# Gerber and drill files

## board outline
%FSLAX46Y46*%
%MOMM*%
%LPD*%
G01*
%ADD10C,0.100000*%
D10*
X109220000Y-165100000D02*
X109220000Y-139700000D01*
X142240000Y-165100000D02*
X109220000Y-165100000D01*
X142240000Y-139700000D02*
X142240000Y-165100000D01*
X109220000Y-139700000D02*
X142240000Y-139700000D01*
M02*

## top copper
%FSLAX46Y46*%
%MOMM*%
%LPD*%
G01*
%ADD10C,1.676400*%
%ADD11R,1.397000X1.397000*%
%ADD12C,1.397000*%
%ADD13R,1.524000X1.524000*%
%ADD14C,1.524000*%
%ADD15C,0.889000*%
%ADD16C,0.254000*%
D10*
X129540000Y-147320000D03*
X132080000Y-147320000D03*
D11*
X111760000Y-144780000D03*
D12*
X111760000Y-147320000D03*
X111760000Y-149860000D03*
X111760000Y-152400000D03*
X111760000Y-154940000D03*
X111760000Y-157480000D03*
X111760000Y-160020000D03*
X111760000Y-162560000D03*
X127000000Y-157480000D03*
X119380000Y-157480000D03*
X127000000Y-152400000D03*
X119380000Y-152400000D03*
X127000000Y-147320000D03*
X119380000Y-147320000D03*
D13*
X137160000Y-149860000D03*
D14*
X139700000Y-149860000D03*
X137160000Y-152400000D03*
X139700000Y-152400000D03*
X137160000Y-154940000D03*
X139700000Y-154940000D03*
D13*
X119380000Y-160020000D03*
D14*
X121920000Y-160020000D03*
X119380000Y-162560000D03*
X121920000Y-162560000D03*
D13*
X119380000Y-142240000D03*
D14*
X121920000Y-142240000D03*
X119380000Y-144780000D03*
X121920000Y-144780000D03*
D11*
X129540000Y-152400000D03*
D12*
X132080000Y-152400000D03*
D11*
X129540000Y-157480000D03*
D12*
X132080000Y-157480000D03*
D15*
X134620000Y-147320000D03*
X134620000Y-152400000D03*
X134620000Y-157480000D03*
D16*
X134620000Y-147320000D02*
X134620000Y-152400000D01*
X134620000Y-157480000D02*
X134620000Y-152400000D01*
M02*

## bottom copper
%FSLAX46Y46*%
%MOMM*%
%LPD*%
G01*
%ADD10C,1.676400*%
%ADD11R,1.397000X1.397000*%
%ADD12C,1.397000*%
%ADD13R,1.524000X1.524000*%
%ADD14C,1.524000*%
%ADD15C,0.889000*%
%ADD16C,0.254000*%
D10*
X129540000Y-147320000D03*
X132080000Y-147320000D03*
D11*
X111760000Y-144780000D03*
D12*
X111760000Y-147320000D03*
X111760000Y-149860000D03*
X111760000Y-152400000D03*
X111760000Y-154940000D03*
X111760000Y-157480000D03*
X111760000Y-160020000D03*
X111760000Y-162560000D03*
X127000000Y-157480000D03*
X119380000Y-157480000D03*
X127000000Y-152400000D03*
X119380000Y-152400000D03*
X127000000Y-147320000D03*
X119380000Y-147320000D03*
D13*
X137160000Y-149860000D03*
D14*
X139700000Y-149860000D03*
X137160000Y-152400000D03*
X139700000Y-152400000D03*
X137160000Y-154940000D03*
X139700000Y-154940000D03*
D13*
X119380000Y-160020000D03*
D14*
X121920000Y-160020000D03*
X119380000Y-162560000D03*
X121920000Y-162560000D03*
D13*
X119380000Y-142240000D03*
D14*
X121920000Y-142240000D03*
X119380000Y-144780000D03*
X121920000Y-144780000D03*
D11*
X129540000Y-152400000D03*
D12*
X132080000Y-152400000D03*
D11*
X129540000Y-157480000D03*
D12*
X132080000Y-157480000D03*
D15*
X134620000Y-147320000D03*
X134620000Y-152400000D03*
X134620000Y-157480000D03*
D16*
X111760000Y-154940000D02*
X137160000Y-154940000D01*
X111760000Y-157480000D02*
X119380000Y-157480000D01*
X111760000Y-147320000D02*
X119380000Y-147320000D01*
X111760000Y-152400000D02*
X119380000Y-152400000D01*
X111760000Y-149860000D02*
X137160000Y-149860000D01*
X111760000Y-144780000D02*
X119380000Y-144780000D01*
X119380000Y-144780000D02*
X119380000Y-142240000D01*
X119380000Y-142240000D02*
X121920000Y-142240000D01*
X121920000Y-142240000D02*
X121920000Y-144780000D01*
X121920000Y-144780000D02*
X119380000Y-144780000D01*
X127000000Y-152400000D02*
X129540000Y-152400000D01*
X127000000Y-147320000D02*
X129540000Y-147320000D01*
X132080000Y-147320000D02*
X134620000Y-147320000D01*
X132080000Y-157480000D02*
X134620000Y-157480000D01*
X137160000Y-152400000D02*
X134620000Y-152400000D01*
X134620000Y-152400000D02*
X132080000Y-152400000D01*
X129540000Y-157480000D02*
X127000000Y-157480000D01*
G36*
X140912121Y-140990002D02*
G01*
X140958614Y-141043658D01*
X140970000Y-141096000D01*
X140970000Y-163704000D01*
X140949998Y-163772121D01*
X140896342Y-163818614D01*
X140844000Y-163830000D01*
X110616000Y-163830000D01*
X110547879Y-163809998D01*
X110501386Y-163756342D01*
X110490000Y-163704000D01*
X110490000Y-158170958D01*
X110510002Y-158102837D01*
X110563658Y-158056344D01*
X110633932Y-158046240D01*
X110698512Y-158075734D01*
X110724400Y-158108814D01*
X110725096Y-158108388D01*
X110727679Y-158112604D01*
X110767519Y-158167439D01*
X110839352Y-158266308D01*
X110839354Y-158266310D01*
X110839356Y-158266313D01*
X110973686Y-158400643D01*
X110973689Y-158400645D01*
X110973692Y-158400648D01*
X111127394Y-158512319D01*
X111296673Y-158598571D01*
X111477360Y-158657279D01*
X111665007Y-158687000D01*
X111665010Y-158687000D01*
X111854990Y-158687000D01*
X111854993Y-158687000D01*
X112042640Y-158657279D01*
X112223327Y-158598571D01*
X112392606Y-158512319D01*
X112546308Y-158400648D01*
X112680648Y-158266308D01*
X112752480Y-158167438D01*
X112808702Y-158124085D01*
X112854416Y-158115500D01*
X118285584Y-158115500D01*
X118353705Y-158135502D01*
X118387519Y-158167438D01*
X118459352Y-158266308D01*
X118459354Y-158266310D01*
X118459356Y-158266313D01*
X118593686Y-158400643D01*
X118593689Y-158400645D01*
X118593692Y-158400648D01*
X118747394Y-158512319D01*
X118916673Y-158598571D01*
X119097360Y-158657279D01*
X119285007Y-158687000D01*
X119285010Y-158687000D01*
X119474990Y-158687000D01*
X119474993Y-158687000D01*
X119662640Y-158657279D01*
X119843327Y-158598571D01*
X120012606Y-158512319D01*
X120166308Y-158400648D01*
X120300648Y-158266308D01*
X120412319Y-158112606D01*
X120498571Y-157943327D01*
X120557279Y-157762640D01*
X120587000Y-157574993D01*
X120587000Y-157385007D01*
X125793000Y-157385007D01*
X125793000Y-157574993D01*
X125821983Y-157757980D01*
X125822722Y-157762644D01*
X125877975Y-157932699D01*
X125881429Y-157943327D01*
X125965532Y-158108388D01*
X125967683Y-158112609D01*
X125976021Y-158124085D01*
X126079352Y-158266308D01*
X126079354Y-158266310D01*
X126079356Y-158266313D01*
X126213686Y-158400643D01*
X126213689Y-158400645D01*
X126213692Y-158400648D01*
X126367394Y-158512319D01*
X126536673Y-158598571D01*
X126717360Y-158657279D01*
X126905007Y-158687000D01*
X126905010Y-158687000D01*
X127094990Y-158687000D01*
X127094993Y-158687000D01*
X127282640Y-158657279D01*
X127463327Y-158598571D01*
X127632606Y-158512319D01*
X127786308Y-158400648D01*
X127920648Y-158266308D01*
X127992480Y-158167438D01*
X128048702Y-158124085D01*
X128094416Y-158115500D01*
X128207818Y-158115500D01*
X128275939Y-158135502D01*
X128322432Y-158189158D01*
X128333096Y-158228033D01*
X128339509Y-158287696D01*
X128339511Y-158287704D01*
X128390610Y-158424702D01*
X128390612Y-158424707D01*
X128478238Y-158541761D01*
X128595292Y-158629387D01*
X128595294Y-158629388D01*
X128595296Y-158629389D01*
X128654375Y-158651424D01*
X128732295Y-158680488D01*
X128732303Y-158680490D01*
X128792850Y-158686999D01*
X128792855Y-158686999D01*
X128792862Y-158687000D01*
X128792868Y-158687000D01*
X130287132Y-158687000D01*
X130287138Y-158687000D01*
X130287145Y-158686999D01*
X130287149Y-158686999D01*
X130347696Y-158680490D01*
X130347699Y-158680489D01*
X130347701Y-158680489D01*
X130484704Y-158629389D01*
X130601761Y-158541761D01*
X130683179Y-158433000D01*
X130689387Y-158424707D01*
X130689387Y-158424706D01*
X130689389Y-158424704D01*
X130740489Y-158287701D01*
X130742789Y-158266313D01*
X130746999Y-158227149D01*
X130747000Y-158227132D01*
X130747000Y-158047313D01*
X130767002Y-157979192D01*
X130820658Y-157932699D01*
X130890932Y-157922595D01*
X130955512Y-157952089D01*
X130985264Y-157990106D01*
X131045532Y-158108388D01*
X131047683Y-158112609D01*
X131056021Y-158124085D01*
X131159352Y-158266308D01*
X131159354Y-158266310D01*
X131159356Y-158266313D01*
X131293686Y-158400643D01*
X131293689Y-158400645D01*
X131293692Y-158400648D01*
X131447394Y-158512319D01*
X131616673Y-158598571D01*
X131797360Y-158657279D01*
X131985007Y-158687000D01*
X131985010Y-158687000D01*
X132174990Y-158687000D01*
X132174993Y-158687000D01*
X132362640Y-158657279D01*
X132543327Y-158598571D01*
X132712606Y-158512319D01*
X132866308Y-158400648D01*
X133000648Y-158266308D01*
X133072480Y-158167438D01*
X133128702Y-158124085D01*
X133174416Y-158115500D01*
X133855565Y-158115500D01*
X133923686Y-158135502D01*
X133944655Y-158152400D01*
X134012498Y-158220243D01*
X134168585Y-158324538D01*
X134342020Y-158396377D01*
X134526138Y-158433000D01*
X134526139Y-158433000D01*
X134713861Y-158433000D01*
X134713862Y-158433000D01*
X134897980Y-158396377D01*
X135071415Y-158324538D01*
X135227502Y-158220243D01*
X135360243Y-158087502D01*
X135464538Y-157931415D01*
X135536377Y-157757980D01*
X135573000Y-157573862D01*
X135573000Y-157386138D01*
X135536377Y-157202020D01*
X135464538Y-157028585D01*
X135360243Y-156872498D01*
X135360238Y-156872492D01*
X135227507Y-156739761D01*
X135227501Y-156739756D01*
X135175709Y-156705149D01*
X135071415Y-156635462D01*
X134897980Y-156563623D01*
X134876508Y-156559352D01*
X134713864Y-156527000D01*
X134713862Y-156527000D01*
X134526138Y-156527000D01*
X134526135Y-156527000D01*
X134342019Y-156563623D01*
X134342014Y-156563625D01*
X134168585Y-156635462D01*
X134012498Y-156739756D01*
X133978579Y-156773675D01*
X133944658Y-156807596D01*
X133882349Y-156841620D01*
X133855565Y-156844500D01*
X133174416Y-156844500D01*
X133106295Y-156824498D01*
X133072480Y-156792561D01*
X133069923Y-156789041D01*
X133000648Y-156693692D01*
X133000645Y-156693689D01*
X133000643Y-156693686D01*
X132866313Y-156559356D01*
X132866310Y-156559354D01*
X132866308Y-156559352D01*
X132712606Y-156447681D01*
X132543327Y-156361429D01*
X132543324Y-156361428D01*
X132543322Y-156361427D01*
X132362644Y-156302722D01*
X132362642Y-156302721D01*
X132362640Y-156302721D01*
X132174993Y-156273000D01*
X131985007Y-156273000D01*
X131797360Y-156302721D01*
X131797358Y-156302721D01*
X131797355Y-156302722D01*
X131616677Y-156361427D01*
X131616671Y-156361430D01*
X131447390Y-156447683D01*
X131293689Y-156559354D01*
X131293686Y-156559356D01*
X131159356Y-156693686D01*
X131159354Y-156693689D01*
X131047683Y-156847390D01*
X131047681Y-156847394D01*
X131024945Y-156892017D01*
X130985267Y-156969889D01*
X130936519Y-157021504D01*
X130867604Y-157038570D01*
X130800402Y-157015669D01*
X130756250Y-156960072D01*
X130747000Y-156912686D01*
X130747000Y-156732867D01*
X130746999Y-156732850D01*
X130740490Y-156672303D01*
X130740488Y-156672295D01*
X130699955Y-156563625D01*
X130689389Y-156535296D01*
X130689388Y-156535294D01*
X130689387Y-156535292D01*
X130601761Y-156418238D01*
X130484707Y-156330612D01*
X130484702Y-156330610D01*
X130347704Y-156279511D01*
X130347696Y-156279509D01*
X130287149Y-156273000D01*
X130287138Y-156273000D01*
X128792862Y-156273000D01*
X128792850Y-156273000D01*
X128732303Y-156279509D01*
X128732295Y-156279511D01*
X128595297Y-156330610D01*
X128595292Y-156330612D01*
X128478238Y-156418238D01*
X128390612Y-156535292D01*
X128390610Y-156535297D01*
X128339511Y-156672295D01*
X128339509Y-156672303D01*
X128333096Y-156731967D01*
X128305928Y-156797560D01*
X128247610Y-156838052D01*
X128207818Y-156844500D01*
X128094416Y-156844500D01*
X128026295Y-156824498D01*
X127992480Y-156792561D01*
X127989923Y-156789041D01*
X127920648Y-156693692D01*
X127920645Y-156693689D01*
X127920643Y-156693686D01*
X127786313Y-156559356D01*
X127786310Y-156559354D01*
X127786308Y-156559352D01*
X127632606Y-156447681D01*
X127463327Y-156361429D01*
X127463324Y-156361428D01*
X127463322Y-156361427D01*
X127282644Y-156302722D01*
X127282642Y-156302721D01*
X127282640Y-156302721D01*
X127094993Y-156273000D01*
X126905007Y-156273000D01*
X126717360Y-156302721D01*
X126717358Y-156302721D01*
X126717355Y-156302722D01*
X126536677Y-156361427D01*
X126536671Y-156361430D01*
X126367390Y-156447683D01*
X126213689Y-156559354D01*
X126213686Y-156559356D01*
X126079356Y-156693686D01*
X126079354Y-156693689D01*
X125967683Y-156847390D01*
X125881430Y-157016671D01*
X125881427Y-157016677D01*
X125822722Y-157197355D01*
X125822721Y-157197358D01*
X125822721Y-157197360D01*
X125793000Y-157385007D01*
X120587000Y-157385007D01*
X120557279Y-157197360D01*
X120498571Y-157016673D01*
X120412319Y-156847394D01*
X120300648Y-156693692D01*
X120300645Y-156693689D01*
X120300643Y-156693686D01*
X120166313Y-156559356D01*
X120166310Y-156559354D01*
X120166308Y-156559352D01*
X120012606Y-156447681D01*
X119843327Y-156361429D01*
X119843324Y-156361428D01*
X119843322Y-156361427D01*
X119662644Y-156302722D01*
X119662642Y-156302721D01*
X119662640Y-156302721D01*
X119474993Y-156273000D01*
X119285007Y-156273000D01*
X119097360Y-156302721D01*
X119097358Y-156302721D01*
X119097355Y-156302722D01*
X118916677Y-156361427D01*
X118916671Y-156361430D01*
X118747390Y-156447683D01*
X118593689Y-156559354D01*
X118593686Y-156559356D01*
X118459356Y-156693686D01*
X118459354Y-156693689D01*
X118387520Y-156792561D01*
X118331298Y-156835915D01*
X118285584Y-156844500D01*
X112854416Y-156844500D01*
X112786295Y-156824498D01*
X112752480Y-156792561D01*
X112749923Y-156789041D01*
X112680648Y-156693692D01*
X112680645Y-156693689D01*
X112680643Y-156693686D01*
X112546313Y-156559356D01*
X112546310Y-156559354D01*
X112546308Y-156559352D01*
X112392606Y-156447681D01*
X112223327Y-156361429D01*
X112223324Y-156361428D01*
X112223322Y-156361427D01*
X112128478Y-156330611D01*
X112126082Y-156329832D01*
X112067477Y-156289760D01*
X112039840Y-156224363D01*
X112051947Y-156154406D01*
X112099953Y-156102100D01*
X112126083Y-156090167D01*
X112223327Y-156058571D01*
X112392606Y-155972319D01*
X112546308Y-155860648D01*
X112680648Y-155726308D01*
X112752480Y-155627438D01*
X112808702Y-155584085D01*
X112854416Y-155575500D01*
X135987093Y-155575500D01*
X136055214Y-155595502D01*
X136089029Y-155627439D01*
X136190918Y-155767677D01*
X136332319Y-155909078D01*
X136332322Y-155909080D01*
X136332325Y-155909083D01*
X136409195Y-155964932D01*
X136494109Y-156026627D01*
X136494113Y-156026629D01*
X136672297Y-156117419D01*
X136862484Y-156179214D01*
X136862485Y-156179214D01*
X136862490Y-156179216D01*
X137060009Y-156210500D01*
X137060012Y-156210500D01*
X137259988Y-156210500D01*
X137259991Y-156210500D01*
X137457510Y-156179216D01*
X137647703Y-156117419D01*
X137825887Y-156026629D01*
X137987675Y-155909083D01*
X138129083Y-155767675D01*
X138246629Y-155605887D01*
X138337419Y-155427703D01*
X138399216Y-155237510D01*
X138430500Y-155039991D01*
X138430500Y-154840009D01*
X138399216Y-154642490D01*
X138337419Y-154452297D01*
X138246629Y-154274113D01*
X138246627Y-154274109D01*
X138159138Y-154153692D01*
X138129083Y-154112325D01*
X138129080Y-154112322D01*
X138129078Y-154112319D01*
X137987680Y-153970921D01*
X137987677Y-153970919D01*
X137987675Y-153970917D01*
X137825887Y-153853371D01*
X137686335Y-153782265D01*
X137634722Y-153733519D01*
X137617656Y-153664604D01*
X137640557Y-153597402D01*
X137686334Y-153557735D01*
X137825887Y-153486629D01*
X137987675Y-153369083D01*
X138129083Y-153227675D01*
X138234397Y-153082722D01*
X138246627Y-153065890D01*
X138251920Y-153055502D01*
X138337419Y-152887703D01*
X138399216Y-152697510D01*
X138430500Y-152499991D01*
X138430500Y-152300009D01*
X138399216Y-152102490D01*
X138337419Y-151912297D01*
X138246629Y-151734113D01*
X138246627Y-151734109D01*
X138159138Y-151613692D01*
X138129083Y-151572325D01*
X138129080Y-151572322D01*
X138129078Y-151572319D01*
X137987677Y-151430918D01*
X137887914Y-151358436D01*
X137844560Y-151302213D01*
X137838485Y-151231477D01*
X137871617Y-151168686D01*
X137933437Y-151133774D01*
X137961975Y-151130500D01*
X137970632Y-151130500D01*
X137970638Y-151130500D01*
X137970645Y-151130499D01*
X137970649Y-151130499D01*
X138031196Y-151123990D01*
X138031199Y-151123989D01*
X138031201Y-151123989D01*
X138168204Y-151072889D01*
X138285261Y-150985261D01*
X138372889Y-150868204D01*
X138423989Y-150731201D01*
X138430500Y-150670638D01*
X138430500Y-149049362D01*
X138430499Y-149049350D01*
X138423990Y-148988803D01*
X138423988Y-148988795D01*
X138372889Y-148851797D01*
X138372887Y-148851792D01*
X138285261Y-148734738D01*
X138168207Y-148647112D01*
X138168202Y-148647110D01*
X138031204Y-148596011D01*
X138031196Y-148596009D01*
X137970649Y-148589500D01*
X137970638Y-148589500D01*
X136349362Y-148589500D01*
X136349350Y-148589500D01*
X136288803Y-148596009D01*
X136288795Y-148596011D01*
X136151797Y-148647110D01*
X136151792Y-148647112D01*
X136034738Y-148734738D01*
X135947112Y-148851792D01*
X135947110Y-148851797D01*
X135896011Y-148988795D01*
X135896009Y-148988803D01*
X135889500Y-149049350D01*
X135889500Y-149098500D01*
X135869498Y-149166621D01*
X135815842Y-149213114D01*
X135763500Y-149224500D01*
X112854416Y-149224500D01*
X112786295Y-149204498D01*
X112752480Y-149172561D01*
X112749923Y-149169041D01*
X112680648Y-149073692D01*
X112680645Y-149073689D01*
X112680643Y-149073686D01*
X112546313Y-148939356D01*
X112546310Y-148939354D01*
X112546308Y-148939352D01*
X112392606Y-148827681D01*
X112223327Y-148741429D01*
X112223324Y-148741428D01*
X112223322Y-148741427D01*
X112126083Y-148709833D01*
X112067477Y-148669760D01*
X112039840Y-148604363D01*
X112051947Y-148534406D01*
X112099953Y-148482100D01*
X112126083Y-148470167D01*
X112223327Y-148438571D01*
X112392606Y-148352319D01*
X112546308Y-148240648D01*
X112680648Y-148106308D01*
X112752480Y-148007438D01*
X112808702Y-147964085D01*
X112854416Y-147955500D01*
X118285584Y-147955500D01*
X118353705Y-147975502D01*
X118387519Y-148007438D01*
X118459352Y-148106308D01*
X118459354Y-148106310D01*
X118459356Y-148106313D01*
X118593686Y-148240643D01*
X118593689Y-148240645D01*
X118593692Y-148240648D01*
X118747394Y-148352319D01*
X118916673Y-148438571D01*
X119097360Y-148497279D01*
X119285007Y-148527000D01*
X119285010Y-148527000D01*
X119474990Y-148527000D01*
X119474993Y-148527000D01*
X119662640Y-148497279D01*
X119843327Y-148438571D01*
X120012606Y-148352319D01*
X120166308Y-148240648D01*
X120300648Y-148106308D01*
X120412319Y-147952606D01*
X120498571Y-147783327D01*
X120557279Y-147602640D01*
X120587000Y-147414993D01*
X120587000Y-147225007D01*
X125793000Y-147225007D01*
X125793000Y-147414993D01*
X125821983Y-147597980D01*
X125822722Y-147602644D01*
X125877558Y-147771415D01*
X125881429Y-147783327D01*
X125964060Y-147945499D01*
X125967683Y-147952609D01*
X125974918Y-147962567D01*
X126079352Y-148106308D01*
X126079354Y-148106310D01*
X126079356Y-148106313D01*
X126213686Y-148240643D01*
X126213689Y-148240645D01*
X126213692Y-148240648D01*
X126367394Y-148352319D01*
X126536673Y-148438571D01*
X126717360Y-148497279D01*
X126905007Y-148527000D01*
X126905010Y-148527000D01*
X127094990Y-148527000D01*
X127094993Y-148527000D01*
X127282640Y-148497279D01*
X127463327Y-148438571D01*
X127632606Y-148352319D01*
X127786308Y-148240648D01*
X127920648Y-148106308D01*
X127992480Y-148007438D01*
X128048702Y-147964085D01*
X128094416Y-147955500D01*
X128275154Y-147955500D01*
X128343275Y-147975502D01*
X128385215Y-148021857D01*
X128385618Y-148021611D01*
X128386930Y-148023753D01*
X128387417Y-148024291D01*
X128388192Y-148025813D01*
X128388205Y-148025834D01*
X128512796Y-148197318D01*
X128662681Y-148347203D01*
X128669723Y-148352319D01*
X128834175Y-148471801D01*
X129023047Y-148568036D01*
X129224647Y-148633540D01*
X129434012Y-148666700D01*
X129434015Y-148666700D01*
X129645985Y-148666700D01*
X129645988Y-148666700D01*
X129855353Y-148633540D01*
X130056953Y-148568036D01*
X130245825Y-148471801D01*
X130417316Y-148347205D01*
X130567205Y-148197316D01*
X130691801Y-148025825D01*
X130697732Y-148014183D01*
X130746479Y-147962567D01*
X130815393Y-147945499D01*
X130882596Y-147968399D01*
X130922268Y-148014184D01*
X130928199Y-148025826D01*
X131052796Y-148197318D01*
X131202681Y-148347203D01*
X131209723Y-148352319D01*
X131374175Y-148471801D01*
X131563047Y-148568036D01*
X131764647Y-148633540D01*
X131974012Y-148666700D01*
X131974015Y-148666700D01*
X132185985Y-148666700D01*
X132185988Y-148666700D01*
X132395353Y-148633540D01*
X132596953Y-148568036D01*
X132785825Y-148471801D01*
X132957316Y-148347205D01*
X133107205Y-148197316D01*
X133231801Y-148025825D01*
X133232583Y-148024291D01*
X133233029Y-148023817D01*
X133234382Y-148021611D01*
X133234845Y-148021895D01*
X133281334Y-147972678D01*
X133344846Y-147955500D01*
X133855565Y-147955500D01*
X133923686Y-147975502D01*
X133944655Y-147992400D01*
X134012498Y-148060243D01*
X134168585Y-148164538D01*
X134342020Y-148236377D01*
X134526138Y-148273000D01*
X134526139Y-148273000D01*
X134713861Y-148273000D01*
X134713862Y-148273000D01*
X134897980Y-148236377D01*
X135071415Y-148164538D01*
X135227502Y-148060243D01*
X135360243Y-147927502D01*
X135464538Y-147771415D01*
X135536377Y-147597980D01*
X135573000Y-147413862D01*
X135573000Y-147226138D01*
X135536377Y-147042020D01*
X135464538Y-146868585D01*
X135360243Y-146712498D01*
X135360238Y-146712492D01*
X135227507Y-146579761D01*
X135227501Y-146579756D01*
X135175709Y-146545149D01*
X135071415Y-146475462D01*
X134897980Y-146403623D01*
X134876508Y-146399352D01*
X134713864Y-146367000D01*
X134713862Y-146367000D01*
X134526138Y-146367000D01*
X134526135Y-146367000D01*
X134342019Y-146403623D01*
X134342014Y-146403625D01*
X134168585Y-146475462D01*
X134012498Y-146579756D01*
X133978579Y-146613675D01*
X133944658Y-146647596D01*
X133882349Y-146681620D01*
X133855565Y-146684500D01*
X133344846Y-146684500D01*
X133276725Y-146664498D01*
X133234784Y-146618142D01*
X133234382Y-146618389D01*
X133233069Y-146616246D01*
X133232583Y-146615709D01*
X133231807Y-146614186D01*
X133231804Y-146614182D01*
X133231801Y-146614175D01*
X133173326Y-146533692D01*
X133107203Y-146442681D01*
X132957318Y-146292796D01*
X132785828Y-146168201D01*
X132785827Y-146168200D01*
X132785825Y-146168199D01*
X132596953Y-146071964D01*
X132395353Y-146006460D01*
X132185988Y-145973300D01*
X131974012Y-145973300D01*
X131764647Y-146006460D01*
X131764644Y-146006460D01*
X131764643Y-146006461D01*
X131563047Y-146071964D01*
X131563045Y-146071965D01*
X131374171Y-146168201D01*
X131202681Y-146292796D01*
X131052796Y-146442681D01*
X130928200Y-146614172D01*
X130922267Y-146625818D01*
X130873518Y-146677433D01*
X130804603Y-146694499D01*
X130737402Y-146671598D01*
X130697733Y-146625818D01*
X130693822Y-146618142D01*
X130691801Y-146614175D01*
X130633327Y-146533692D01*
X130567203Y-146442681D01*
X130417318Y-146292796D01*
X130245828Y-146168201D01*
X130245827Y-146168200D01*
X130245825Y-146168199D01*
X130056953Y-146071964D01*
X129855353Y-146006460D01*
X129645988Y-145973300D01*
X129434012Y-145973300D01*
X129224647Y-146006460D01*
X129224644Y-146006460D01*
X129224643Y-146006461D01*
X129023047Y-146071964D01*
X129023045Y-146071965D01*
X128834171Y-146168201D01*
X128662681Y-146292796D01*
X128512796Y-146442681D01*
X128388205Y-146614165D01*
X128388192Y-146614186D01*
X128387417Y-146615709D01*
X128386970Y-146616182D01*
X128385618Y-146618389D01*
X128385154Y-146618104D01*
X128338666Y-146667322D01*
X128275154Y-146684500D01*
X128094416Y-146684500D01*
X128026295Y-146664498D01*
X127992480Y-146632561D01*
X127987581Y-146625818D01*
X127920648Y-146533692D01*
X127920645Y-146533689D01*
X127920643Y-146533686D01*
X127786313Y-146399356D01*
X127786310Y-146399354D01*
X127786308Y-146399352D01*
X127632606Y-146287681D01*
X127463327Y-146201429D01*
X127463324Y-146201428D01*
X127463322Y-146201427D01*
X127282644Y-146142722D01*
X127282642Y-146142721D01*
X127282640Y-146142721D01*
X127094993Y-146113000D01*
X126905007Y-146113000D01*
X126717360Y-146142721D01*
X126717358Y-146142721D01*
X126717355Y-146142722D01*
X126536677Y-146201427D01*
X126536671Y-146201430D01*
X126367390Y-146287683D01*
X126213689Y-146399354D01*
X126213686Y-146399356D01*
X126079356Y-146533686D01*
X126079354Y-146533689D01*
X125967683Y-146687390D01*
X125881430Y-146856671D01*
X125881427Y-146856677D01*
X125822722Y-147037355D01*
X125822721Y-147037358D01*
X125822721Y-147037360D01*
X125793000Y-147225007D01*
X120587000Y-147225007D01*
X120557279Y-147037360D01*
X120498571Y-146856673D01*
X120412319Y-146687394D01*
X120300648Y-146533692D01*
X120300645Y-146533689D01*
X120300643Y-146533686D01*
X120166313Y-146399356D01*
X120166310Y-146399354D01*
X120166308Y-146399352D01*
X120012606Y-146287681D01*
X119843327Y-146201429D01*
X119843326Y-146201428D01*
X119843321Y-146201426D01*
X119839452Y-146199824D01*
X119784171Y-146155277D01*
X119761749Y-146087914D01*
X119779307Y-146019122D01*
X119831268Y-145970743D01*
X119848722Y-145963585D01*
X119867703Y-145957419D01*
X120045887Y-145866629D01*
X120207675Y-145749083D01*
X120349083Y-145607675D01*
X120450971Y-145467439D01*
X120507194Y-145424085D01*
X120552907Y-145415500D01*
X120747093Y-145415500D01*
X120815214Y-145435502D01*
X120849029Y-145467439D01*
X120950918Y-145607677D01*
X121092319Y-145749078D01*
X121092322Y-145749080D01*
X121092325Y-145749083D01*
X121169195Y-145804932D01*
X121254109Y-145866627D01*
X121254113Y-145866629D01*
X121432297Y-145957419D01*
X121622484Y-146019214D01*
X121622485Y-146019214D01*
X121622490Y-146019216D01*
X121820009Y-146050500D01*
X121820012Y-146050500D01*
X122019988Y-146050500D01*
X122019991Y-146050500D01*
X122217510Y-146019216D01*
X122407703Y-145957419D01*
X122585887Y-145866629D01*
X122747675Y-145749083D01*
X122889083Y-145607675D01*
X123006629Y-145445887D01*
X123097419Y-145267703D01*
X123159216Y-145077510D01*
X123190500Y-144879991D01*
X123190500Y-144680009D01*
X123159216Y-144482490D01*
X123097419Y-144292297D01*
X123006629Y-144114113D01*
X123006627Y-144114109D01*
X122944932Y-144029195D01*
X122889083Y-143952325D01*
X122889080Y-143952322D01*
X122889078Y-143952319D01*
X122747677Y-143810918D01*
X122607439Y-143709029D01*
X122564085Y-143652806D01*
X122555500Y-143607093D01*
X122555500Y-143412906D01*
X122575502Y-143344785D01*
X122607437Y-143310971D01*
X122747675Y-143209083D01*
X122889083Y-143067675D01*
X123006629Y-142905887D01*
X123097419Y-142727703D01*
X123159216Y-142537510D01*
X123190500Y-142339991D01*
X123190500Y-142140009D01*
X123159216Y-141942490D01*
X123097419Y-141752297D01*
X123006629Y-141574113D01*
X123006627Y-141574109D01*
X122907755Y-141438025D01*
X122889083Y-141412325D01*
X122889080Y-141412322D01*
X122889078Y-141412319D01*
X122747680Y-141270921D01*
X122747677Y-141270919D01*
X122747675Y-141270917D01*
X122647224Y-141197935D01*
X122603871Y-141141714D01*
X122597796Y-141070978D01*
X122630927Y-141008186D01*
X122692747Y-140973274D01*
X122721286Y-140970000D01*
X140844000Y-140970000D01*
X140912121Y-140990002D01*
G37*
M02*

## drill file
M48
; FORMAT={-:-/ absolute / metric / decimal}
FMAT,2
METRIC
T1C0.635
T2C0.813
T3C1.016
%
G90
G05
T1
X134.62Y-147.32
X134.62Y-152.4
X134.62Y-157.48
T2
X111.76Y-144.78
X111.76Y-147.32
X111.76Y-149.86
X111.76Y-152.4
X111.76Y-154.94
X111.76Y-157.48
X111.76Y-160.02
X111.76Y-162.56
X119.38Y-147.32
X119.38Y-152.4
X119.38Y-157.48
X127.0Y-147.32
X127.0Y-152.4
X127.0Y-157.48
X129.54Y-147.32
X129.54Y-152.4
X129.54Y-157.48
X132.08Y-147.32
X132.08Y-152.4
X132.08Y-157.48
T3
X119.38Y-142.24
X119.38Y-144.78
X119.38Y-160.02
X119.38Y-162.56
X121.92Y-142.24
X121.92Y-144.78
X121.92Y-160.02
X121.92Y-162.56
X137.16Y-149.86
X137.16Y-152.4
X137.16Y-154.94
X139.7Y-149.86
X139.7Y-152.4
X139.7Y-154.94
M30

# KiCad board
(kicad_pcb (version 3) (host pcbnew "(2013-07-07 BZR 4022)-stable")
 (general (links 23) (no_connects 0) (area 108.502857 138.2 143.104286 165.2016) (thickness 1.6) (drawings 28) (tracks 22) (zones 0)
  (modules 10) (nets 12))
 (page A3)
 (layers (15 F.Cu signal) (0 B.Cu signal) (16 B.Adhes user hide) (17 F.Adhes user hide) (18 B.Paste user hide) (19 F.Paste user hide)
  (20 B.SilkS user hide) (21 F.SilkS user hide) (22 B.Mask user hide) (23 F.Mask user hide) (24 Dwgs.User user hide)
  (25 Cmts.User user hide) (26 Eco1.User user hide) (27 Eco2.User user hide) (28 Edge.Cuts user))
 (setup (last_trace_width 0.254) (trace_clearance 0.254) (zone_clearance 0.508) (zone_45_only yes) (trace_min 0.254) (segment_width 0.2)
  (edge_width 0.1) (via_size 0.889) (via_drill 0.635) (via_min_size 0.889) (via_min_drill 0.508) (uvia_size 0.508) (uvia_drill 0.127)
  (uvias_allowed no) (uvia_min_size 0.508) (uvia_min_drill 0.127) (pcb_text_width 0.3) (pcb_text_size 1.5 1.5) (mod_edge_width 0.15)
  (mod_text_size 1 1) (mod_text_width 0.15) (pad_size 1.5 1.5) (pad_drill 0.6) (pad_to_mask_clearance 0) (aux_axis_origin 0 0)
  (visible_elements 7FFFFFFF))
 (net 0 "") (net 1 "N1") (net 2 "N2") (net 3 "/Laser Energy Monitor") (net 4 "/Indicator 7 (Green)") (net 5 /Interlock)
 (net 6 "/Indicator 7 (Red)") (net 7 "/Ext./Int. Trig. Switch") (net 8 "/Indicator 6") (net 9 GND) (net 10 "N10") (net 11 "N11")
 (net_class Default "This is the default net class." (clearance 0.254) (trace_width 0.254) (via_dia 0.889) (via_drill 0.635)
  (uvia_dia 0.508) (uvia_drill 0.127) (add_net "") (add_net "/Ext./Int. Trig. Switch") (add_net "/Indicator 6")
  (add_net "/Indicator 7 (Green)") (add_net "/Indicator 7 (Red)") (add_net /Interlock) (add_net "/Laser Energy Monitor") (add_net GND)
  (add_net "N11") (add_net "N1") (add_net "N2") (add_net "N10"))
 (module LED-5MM (layer F.Cu) (at 130.81 147.32)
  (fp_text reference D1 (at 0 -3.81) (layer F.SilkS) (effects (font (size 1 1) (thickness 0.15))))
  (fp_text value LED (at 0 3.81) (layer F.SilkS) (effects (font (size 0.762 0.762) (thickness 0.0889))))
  (pad 1 thru_hole circle (at -1.27 0) (size 1.6764 1.6764) (drill 0.8128) (layers *.Cu *.Mask F.SilkS) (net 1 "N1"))
  (pad 2 thru_hole circle (at 1.27 0) (size 1.6764 1.6764) (drill 0.8128) (layers *.Cu *.Mask F.SilkS) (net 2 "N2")))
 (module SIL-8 (layer F.Cu) (at 111.76 153.67 270)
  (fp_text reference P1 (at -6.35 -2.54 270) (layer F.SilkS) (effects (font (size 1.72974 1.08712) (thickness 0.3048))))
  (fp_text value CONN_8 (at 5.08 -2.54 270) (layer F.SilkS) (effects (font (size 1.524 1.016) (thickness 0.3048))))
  (pad 1 thru_hole rect (at -8.89 0 270) (size 1.397 1.397) (drill 0.8128) (layers *.Cu *.Mask F.SilkS) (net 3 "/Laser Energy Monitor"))
  (pad 2 thru_hole circle (at -6.35 0 270) (size 1.397 1.397) (drill 0.8128) (layers *.Cu *.Mask F.SilkS) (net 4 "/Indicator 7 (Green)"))
  (pad 3 thru_hole circle (at -3.81 0 270) (size 1.397 1.397) (drill 0.8128) (layers *.Cu *.Mask F.SilkS) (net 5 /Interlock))
  (pad 4 thru_hole circle (at -1.27 0 270) (size 1.397 1.397) (drill 0.8128) (layers *.Cu *.Mask F.SilkS) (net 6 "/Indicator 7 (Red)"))
  (pad 5 thru_hole circle (at 1.27 0 270) (size 1.397 1.397) (drill 0.8128) (layers *.Cu *.Mask F.SilkS) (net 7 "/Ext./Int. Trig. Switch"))
  (pad 6 thru_hole circle (at 3.81 0 270) (size 1.397 1.397) (drill 0.8128) (layers *.Cu *.Mask F.SilkS) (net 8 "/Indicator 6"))
  (pad 7 thru_hole circle (at 6.35 0 270) (size 1.397 1.397) (drill 0.8128) (layers *.Cu *.Mask F.SilkS) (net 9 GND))
  (pad 8 thru_hole circle (at 8.89 0 270) (size 1.397 1.397) (drill 0.8128) (layers *.Cu *.Mask F.SilkS) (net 9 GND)))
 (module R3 (layer F.Cu) (at 123.19 157.48 180) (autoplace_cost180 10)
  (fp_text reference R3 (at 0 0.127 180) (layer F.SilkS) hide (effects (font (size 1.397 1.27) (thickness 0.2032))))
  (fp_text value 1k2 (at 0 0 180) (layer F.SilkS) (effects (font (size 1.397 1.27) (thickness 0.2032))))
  (pad 1 thru_hole circle (at -3.81 0 180) (size 1.397 1.397) (drill 0.8128) (layers *.Cu *.Mask F.SilkS) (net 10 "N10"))
  (pad 2 thru_hole circle (at 3.81 0 180) (size 1.397 1.397) (drill 0.8128) (layers *.Cu *.Mask F.SilkS) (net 8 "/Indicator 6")))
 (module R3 (layer F.Cu) (at 123.19 152.4 180) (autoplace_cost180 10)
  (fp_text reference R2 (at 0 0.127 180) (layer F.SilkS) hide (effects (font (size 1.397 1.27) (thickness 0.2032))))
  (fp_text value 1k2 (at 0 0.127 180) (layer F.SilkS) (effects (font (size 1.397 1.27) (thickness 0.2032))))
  (pad 1 thru_hole circle (at -3.81 0 180) (size 1.397 1.397) (drill 0.8128) (layers *.Cu *.Mask F.SilkS) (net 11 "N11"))
  (pad 2 thru_hole circle (at 3.81 0 180) (size 1.397 1.397) (drill 0.8128) (layers *.Cu *.Mask F.SilkS) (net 6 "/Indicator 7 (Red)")))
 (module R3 (layer F.Cu) (at 123.19 147.32 180) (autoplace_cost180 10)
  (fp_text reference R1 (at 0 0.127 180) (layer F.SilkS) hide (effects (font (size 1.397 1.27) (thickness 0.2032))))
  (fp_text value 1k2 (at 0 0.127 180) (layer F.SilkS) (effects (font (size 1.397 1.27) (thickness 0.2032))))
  (pad 1 thru_hole circle (at -3.81 0 180) (size 1.397 1.397) (drill 0.8128) (layers *.Cu *.Mask F.SilkS) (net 1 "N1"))
  (pad 2 thru_hole circle (at 3.81 0 180) (size 1.397 1.397) (drill 0.8128) (layers *.Cu *.Mask F.SilkS) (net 4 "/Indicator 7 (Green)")))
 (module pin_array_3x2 (layer F.Cu) (at 138.43 152.4 270)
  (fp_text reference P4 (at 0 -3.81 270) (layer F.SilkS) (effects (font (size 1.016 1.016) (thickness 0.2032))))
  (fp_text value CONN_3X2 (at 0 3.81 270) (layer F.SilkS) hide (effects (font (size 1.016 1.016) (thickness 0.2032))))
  (pad 1 thru_hole rect (at -2.54 1.27 270) (size 1.524 1.524) (drill 1.016) (layers *.Cu *.Mask F.SilkS) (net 5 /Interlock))
  (pad 2 thru_hole circle (at -2.54 -1.27 270) (size 1.524 1.524) (drill 1.016) (layers *.Cu *.Mask F.SilkS) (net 9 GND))
  (pad 3 thru_hole circle (at 0 1.27 270) (size 1.524 1.524) (drill 1.016) (layers *.Cu *.Mask F.SilkS) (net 2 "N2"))
  (pad 4 thru_hole circle (at 0 -1.27 270) (size 1.524 1.524) (drill 1.016) (layers *.Cu *.Mask F.SilkS) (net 9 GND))
  (pad 5 thru_hole circle (at 2.54 1.27 270) (size 1.524 1.524) (drill 1.016) (layers *.Cu *.Mask F.SilkS) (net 7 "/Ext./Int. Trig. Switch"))
  (pad 6 thru_hole circle (at 2.54 -1.27 270) (size 1.524 1.524) (drill 1.016) (layers *.Cu *.Mask F.SilkS) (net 9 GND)))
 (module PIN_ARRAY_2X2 (layer F.Cu) (at 120.65 161.29 270)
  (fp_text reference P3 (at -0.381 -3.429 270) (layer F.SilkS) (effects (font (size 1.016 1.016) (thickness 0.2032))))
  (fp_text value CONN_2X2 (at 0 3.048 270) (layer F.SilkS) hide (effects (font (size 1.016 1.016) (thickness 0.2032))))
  (pad 1 thru_hole rect (at -1.27 1.27 270) (size 1.524 1.524) (drill 1.016) (layers *.Cu *.Mask F.SilkS) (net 9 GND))
  (pad 2 thru_hole circle (at -1.27 -1.27 270) (size 1.524 1.524) (drill 1.016) (layers *.Cu *.Mask F.SilkS) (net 9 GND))
  (pad 3 thru_hole circle (at 1.27 1.27 270) (size 1.524 1.524) (drill 1.016) (layers *.Cu *.Mask F.SilkS) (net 9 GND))
  (pad 4 thru_hole circle (at 1.27 -1.27 270) (size 1.524 1.524) (drill 1.016) (layers *.Cu *.Mask F.SilkS) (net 9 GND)))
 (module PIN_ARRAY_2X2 (layer F.Cu) (at 120.65 143.51 270)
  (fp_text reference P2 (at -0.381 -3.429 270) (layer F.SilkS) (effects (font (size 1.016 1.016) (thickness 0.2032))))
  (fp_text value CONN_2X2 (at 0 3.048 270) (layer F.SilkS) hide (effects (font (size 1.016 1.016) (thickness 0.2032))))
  (pad 1 thru_hole rect (at -1.27 1.27 270) (size 1.524 1.524) (drill 1.016) (layers *.Cu *.Mask F.SilkS) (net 3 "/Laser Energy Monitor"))
  (pad 2 thru_hole circle (at -1.27 -1.27 270) (size 1.524 1.524) (drill 1.016) (layers *.Cu *.Mask F.SilkS) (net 3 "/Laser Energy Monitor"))
  (pad 3 thru_hole circle (at 1.27 1.27 270) (size 1.524 1.524) (drill 1.016) (layers *.Cu *.Mask F.SilkS) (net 3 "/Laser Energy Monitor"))
  (pad 4 thru_hole circle (at 1.27 -1.27 270) (size 1.524 1.524) (drill 1.016) (layers *.Cu *.Mask F.SilkS) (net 3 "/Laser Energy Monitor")))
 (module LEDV (layer F.Cu) (at 130.81 152.4)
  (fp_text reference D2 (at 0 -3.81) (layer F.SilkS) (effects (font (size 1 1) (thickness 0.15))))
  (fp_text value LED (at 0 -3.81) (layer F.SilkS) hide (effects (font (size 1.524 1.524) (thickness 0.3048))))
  (pad 1 thru_hole rect (at -1.27 0) (size 1.397 1.397) (drill 0.8128) (layers *.Cu *.Mask F.SilkS) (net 11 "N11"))
  (pad 2 thru_hole circle (at 1.27 0) (size 1.397 1.397) (drill 0.8128) (layers *.Cu *.Mask F.SilkS) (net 2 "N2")))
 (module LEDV (layer F.Cu) (at 130.81 157.48)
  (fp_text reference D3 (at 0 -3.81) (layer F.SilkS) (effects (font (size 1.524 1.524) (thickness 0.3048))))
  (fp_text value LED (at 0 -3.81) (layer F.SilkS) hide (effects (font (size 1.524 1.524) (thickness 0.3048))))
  (pad 1 thru_hole rect (at -1.27 0) (size 1.397 1.397) (drill 0.8128) (layers *.Cu *.Mask F.SilkS) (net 10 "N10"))
  (pad 2 thru_hole circle (at 1.27 0) (size 1.397 1.397) (drill 0.8128) (layers *.Cu *.Mask F.SilkS) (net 2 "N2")))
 (gr_line (start 109.22 165.1) (end 109.22 139.7) (angle 90) (layer Edge.Cuts) (width 0.1))
 (gr_line (start 142.24 165.1) (end 109.22 165.1) (angle 90) (layer Edge.Cuts) (width 0.1))
 (gr_line (start 142.24 139.7) (end 142.24 165.1) (angle 90) (layer Edge.Cuts) (width 0.1))
 (gr_line (start 109.22 139.7) (end 142.24 139.7) (angle 90) (layer Edge.Cuts) (width 0.1))
 (segment (start 111.76 154.94) (end 137.16 154.94) (width 0.254) (layer B.Cu) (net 7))
 (segment (start 111.76 157.48) (end 119.38 157.48) (width 0.254) (layer B.Cu) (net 8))
 (segment (start 111.76 147.32) (end 119.38 147.32) (width 0.254) (layer B.Cu) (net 4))
 (segment (start 111.76 152.4) (end 119.38 152.4) (width 0.254) (layer B.Cu) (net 6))
 (segment (start 111.76 149.86) (end 137.16 149.86) (width 0.254) (layer B.Cu) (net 5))
 (segment (start 111.76 144.78) (end 119.38 144.78) (width 0.254) (layer B.Cu) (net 3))
 (segment (start 119.38 144.78) (end 119.38 142.24) (width 0.254) (layer B.Cu) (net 3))
 (segment (start 119.38 142.24) (end 121.92 142.24) (width 0.254) (layer B.Cu) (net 3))
 (segment (start 121.92 142.24) (end 121.92 144.78) (width 0.254) (layer B.Cu) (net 3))
 (segment (start 121.92 144.78) (end 119.38 144.78) (width 0.254) (layer B.Cu) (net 3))
 (segment (start 127 152.4) (end 129.54 152.4) (width 0.254) (layer B.Cu) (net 11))
 (segment (start 127 147.32) (end 129.54 147.32) (width 0.254) (layer B.Cu) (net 1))
 (segment (start 132.08 147.32) (end 134.62 147.32) (width 0.254) (layer B.Cu) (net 2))
 (segment (start 134.62 147.32) (end 134.62 152.4) (width 0.254) (layer F.Cu) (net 2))
 (via (at 134.62 147.32) (size 0.889) (layers F.Cu B.Cu) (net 2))
 (segment (start 132.08 157.48) (end 134.62 157.48) (width 0.254) (layer B.Cu) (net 2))
 (via (at 134.62 152.4) (size 0.889) (layers F.Cu B.Cu) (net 2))
 (segment (start 134.62 157.48) (end 134.62 152.4) (width 0.254) (layer F.Cu) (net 2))
 (via (at 134.62 157.48) (size 0.889) (layers F.Cu B.Cu) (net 2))
 (segment (start 137.16 152.4) (end 134.62 152.4) (width 0.254) (layer B.Cu) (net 2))
 (segment (start 134.62 152.4) (end 132.08 152.4) (width 0.254) (layer B.Cu) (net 2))
 (segment (start 129.54 157.48) (end 127 157.48) (width 0.254) (layer B.Cu) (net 10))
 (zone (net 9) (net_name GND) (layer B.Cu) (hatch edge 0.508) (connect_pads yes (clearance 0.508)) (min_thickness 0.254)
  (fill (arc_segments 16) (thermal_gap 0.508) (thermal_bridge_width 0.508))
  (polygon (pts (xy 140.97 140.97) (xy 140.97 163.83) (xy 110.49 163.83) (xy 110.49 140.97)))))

